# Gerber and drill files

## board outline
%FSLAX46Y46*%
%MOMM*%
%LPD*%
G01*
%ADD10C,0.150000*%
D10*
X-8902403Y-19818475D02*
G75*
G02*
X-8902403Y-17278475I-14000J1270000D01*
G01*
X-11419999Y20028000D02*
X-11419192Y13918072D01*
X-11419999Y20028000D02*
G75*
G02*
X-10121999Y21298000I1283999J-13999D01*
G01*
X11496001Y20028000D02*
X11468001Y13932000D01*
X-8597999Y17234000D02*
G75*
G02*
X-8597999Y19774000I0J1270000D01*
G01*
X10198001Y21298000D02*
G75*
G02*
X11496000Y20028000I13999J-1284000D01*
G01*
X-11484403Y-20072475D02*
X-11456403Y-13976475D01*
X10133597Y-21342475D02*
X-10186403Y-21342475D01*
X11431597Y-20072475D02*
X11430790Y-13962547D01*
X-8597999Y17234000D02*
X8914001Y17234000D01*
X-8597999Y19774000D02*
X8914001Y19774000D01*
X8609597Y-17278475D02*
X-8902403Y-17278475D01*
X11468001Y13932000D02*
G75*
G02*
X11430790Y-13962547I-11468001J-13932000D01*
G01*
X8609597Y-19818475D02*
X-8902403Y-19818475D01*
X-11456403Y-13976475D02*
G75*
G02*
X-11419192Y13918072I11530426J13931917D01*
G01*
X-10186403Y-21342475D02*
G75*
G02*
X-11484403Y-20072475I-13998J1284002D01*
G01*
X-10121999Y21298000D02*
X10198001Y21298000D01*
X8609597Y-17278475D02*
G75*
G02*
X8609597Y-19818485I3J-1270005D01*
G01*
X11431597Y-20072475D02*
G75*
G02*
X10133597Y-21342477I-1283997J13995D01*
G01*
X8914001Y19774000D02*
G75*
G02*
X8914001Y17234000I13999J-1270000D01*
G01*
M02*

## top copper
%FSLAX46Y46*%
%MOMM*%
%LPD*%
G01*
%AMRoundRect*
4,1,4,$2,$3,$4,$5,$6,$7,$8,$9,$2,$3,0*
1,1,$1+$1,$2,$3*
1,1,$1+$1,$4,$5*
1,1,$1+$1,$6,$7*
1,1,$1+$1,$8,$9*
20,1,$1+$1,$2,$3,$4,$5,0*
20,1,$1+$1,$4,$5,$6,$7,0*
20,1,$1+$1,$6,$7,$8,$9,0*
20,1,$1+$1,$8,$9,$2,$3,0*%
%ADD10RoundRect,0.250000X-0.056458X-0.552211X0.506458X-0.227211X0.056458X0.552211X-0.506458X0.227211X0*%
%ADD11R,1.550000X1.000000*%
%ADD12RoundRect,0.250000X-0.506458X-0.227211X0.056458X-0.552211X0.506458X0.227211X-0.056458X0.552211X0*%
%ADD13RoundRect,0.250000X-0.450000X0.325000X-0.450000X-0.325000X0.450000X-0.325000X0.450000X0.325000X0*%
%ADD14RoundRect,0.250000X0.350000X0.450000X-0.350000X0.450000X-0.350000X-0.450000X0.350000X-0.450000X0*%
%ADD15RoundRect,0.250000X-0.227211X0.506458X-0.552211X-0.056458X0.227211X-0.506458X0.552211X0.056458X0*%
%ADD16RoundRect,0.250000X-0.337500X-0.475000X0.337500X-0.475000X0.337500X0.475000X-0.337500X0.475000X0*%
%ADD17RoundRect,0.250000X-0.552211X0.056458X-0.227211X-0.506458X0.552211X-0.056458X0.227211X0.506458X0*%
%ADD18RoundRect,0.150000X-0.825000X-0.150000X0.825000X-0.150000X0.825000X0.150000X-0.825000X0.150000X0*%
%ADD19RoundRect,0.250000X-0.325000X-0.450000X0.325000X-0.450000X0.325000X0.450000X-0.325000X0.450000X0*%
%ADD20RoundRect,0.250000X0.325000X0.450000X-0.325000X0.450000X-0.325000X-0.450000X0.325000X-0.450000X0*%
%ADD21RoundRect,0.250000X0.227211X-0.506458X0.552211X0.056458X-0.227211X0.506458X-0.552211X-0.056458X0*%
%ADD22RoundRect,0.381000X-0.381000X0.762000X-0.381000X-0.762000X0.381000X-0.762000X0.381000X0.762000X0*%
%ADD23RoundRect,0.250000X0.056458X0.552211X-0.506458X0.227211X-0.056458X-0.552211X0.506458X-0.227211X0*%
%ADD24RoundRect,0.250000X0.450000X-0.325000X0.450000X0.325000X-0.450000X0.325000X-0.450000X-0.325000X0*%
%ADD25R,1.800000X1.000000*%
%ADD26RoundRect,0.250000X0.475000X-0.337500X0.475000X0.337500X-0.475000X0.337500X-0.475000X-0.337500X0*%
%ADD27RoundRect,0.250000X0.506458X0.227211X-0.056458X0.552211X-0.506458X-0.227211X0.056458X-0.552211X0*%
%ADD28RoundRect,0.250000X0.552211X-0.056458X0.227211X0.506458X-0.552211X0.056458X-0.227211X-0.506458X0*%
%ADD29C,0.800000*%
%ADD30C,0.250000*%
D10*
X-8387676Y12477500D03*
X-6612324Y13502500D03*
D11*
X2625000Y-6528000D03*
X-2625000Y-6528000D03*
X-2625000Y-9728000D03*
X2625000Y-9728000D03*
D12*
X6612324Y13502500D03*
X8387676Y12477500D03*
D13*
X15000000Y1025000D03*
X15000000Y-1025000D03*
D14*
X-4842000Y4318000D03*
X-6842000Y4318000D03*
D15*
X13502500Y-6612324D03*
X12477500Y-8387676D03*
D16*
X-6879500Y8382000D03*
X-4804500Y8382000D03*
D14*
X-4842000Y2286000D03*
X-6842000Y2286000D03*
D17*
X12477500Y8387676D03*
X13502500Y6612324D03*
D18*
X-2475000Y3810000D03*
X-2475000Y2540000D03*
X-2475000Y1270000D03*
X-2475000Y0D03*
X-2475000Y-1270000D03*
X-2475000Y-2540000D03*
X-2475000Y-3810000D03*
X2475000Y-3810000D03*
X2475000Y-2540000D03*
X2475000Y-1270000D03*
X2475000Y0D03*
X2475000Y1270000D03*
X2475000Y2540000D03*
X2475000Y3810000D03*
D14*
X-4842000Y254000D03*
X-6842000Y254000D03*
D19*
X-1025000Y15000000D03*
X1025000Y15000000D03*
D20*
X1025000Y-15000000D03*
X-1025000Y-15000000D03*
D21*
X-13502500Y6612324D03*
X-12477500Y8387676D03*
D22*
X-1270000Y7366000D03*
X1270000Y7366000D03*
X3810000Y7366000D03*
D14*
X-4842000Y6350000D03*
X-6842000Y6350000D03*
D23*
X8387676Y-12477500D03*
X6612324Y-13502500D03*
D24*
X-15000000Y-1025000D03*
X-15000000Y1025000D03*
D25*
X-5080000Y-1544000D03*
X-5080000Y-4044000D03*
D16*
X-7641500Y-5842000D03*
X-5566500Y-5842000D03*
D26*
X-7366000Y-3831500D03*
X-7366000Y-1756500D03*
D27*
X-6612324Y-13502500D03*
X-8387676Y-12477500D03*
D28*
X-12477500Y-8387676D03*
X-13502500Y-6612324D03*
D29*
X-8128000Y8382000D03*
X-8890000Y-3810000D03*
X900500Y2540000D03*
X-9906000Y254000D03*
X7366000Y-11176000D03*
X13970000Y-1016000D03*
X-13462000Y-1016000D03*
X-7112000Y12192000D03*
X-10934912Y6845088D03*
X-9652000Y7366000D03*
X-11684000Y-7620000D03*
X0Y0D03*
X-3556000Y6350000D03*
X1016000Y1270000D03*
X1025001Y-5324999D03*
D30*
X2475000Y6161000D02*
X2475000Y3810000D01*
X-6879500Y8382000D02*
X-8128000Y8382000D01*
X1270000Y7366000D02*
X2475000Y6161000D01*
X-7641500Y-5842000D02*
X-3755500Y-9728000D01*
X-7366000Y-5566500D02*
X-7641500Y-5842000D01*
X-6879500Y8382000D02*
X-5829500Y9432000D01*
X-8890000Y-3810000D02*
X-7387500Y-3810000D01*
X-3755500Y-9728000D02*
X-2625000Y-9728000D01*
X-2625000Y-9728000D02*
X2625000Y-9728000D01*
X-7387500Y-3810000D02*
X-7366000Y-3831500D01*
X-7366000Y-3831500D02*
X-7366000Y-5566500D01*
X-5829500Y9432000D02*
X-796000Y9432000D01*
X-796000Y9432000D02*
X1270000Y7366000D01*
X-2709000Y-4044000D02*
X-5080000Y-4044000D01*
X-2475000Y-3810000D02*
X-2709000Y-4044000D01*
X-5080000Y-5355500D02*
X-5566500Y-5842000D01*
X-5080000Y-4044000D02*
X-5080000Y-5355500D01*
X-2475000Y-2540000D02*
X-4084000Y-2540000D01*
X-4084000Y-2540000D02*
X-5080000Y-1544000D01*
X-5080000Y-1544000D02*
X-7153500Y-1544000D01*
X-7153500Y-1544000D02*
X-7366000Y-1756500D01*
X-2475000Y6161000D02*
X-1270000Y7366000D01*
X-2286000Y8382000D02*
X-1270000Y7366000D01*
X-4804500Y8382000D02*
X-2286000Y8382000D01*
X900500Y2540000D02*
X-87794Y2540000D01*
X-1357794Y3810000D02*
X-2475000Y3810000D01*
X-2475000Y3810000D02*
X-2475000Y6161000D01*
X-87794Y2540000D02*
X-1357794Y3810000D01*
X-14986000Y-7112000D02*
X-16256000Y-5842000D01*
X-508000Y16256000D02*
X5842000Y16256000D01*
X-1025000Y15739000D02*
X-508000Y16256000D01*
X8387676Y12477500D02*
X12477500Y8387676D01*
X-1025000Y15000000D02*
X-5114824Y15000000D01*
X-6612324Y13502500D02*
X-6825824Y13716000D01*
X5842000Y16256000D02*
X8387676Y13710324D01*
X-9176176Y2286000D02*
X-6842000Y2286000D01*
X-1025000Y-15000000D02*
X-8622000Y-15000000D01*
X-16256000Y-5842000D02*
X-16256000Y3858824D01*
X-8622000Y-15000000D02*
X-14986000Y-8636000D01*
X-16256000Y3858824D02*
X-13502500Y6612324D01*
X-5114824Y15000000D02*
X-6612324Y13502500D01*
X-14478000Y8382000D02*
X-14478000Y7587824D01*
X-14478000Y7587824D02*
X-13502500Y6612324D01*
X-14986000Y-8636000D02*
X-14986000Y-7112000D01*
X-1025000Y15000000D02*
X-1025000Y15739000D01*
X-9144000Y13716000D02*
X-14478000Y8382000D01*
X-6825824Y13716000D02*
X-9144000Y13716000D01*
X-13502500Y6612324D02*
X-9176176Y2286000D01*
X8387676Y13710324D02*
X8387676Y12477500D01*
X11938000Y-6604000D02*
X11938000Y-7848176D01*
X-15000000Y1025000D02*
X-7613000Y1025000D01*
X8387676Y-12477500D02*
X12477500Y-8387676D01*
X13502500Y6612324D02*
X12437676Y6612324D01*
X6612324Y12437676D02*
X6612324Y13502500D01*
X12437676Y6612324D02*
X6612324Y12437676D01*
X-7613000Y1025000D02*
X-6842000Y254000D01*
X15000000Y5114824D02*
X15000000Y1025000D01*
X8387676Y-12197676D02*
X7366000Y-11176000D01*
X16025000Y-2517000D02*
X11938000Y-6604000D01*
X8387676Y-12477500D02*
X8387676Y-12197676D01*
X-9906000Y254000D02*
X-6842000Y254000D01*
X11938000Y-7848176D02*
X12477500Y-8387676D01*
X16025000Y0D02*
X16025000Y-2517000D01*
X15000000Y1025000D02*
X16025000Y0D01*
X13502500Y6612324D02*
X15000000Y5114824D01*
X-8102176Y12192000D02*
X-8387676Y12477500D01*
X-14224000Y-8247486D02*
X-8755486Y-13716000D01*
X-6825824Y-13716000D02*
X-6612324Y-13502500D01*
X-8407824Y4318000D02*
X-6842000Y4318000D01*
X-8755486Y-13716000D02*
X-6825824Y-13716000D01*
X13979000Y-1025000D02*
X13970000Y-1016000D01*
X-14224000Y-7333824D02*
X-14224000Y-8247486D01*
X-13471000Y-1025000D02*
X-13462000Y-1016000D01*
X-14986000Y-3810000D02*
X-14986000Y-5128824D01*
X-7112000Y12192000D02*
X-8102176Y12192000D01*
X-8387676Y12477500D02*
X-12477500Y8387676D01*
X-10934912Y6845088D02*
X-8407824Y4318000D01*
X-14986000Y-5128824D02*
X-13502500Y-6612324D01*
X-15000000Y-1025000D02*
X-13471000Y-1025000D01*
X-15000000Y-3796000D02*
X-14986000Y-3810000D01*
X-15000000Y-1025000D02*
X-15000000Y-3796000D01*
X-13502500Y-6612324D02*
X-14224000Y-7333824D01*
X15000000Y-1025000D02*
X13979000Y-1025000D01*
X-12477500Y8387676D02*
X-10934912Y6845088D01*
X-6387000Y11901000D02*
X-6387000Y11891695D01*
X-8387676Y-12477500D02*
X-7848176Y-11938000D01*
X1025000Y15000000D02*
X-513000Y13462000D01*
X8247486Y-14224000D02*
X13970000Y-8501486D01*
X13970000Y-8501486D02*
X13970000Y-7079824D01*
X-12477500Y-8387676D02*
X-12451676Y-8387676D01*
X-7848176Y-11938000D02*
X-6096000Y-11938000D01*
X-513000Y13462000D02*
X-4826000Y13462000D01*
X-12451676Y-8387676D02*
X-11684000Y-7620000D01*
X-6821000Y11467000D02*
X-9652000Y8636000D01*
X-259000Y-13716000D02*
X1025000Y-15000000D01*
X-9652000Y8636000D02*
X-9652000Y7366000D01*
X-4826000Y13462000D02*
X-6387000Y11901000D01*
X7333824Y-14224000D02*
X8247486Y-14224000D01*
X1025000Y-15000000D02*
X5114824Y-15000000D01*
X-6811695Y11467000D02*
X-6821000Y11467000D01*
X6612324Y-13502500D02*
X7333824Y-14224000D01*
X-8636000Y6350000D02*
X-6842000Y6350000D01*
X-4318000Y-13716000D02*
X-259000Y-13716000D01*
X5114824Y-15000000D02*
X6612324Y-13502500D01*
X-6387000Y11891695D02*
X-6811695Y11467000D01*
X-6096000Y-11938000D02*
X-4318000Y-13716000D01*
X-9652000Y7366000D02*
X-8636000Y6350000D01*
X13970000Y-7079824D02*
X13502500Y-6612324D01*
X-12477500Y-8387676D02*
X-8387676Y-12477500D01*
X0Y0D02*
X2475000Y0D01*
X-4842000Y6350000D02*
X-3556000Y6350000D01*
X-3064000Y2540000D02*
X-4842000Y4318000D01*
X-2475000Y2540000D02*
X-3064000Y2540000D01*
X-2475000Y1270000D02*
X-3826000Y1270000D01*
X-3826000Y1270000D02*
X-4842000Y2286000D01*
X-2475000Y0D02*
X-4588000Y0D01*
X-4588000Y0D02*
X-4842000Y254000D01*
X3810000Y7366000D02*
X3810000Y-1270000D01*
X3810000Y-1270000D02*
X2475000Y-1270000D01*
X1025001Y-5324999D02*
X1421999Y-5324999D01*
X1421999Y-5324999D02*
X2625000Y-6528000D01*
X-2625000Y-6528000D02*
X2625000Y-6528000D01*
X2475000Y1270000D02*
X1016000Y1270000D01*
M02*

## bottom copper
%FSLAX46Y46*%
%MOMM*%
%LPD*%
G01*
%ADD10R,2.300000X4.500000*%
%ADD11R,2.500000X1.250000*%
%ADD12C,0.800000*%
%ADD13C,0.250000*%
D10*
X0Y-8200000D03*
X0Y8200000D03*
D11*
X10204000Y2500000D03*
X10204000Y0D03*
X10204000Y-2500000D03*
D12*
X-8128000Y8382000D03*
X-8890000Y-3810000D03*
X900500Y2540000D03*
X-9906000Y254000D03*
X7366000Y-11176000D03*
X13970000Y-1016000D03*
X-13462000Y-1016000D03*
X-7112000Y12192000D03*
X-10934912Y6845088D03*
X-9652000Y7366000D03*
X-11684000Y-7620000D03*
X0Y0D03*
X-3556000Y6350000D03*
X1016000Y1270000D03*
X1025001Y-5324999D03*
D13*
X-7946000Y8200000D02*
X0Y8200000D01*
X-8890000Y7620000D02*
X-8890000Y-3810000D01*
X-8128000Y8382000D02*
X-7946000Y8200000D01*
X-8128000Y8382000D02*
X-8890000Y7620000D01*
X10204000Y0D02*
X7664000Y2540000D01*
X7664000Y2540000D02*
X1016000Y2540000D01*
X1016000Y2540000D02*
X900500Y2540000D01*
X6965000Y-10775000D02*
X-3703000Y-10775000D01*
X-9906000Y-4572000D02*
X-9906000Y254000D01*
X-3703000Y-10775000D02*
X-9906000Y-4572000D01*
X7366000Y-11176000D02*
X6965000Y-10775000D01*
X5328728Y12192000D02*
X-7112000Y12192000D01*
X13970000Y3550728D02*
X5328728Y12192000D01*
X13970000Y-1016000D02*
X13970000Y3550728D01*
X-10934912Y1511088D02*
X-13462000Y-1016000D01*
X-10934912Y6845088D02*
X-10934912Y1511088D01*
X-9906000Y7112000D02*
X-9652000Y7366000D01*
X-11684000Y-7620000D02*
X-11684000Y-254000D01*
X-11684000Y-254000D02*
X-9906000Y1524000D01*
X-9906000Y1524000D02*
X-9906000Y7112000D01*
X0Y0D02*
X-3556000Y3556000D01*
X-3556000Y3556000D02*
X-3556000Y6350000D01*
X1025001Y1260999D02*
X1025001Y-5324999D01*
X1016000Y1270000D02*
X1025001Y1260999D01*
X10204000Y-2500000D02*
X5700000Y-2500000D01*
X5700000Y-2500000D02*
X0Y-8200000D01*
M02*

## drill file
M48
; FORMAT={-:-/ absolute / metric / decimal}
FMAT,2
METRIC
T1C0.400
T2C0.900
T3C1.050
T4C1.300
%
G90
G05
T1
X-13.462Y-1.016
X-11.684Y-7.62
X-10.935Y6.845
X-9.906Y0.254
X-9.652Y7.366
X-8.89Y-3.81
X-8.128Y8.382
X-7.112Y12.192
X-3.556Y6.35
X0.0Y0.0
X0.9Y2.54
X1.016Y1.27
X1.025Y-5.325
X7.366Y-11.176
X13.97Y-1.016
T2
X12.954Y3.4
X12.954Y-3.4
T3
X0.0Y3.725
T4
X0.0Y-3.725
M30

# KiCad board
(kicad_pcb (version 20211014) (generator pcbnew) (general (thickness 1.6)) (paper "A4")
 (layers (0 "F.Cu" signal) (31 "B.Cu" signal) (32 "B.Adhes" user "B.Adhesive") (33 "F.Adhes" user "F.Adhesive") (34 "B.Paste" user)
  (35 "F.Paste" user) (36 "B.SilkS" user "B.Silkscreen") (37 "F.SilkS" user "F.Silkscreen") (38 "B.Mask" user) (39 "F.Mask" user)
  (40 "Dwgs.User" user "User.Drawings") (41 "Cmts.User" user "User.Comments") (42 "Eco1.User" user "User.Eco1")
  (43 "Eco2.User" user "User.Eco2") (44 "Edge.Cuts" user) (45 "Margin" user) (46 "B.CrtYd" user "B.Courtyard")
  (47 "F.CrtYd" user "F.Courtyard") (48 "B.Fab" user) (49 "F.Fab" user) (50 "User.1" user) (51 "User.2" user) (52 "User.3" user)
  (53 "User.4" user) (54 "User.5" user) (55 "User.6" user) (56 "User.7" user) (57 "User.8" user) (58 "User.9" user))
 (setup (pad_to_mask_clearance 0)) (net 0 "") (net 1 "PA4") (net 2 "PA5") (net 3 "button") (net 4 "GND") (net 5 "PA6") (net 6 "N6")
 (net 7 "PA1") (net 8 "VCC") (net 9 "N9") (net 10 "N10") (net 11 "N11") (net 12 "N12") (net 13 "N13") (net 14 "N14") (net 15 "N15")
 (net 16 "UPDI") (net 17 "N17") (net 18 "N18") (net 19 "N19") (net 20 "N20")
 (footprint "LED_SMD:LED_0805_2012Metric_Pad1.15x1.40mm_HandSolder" (layer "F.Cu") (at -7.5 -12.99 30)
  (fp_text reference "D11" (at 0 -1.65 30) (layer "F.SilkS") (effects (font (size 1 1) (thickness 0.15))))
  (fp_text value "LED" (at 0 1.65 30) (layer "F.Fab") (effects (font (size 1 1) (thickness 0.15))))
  (pad "1" smd roundrect (at -1.025 0 30) (size 1.15 1.4) (layers "F.Cu" "F.Paste" "F.Mask") (roundrect_rratio 0.217391) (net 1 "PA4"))
  (pad "2" smd roundrect (at 1.025 0 30) (size 1.15 1.4) (layers "F.Cu" "F.Paste" "F.Mask") (roundrect_rratio 0.217391) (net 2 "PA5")))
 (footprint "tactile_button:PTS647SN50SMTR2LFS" (layer "F.Cu") (at 0 8.128 180)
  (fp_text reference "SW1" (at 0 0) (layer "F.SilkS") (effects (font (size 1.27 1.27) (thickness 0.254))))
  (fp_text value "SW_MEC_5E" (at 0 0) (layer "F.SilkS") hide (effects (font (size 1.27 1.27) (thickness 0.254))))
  (pad "1" smd rect locked (at -2.625 1.6 270) (size 1 1.55) (layers "F.Cu" "F.Paste" "F.Mask") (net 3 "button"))
  (pad "2" smd rect locked (at 2.625 1.6 270) (size 1 1.55) (layers "F.Cu" "F.Paste" "F.Mask") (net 3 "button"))
  (pad "3" smd rect locked (at 2.625 -1.6 270) (size 1 1.55) (layers "F.Cu" "F.Paste" "F.Mask") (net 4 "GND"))
  (pad "4" smd rect locked (at -2.625 -1.6 270) (size 1 1.55) (layers "F.Cu" "F.Paste" "F.Mask") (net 4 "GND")))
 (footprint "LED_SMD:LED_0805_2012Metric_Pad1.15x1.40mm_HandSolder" (layer "F.Cu") (at 7.5 -12.99 -30)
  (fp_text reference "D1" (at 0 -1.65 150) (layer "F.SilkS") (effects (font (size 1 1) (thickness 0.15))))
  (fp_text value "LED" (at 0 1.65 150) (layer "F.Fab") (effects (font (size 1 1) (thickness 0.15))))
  (pad "1" smd roundrect (at -1.025 0 330) (size 1.15 1.4) (layers "F.Cu" "F.Paste" "F.Mask") (roundrect_rratio 0.217391) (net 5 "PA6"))
  (pad "2" smd roundrect (at 1.025 0 330) (size 1.15 1.4) (layers "F.Cu" "F.Paste" "F.Mask") (roundrect_rratio 0.217391) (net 2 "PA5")))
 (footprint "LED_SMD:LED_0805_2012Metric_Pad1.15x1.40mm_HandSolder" (layer "F.Cu") (at 15 0 -90)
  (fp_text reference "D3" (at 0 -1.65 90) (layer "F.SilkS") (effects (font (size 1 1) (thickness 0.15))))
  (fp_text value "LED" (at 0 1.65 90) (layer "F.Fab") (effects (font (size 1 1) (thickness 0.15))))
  (pad "1" smd roundrect (at -1.025 0 270) (size 1.15 1.4) (layers "F.Cu" "F.Paste" "F.Mask") (roundrect_rratio 0.217391) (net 5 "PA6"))
  (pad "2" smd roundrect (at 1.025 0 270) (size 1.15 1.4) (layers "F.Cu" "F.Paste" "F.Mask") (roundrect_rratio 0.217391) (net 1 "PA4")))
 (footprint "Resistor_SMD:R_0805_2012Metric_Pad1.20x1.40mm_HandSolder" (layer "F.Cu") (at -5.842 -4.318 180)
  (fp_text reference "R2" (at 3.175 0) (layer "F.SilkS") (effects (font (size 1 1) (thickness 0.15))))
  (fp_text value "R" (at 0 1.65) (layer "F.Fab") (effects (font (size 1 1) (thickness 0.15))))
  (pad "1" smd roundrect (at -1 0 180) (size 1.2 1.4) (layers "F.Cu" "F.Paste" "F.Mask") (roundrect_rratio 0.208333) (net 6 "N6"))
  (pad "2" smd roundrect (at 1 0 180) (size 1.2 1.4) (layers "F.Cu" "F.Paste" "F.Mask") (roundrect_rratio 0.208333) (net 1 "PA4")))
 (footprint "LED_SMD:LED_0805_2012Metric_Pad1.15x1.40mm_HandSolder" (layer "F.Cu") (at 12.99 7.5 -120)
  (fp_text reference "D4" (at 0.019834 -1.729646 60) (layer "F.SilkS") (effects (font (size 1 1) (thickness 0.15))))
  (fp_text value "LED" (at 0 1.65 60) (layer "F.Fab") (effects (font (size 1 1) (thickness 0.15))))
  (pad "1" smd roundrect (at -1.025 0 240) (size 1.15 1.4) (layers "F.Cu" "F.Paste" "F.Mask") (roundrect_rratio 0.217391) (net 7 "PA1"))
  (pad "2" smd roundrect (at 1.025 0 240) (size 1.15 1.4) (layers "F.Cu" "F.Paste" "F.Mask") (roundrect_rratio 0.217391) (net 5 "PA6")))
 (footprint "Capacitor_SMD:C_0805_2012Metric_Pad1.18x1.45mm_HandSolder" (layer "F.Cu") (at -5.842 -8.382)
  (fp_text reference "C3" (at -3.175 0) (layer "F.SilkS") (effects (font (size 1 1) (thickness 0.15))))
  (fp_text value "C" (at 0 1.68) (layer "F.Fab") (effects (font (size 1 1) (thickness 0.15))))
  (pad "1" smd roundrect (at -1.0375 0) (size 1.175 1.45) (layers "F.Cu" "F.Paste" "F.Mask") (roundrect_rratio 0.212766) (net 4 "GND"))
  (pad "2" smd roundrect (at 1.0375 0) (size 1.175 1.45) (layers "F.Cu" "F.Paste" "F.Mask") (roundrect_rratio 0.212766) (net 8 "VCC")))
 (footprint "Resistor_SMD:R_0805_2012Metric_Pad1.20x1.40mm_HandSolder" (layer "F.Cu") (at -5.842 -2.286 180)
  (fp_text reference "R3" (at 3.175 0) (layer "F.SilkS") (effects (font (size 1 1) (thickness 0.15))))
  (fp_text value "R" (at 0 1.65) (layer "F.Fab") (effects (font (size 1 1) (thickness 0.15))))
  (pad "1" smd roundrect (at -1 0 180) (size 1.2 1.4) (layers "F.Cu" "F.Paste" "F.Mask") (roundrect_rratio 0.208333) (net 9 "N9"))
  (pad "2" smd roundrect (at 1 0 180) (size 1.2 1.4) (layers "F.Cu" "F.Paste" "F.Mask") (roundrect_rratio 0.208333) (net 2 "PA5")))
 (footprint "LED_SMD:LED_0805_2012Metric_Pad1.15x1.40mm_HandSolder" (layer "F.Cu") (at 12.99 -7.5 -60)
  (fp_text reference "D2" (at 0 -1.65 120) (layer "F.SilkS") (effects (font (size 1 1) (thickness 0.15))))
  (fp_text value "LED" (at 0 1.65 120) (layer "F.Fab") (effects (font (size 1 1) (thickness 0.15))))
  (pad "1" smd roundrect (at -1.025 0 300) (size 1.15 1.4) (layers "F.Cu" "F.Paste" "F.Mask") (roundrect_rratio 0.217391) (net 2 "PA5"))
  (pad "2" smd roundrect (at 1.025 0 300) (size 1.15 1.4) (layers "F.Cu" "F.Paste" "F.Mask") (roundrect_rratio 0.217391) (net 5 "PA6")))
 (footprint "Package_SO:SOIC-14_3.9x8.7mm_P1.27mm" (layer "F.Cu") (at 0 0)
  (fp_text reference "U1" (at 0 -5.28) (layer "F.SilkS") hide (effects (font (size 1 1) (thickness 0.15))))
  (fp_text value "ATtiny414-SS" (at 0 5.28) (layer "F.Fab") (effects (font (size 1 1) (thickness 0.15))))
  (pad "1" smd roundrect (at -2.475 -3.81) (size 1.95 0.6) (layers "F.Cu" "F.Paste" "F.Mask") (roundrect_rratio 0.25) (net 8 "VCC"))
  (pad "2" smd roundrect (at -2.475 -2.54) (size 1.95 0.6) (layers "F.Cu" "F.Paste" "F.Mask") (roundrect_rratio 0.25) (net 6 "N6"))
  (pad "3" smd roundrect (at -2.475 -1.27) (size 1.95 0.6) (layers "F.Cu" "F.Paste" "F.Mask") (roundrect_rratio 0.25) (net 9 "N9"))
  (pad "4" smd roundrect (at -2.475 0) (size 1.95 0.6) (layers "F.Cu" "F.Paste" "F.Mask") (roundrect_rratio 0.25) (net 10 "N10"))
  (pad "5" smd roundrect (at -2.475 1.27) (size 1.95 0.6) (layers "F.Cu" "F.Paste" "F.Mask") (roundrect_rratio 0.25) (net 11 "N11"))
  (pad "6" smd roundrect (at -2.475 2.54) (size 1.95 0.6) (layers "F.Cu" "F.Paste" "F.Mask") (roundrect_rratio 0.25) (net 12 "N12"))
  (pad "7" smd roundrect (at -2.475 3.81) (size 1.95 0.6) (layers "F.Cu" "F.Paste" "F.Mask") (roundrect_rratio 0.25) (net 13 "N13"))
  (pad "8" smd roundrect (at 2.475 3.81) (size 1.95 0.6) (layers "F.Cu" "F.Paste" "F.Mask") (roundrect_rratio 0.25) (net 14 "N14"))
  (pad "9" smd roundrect (at 2.475 2.54) (size 1.95 0.6) (layers "F.Cu" "F.Paste" "F.Mask") (roundrect_rratio 0.25) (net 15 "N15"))
  (pad "10" smd roundrect (at 2.475 1.27) (size 1.95 0.6) (layers "F.Cu" "F.Paste" "F.Mask") (roundrect_rratio 0.25) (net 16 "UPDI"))
  (pad "11" smd roundrect (at 2.475 0) (size 1.95 0.6) (layers "F.Cu" "F.Paste" "F.Mask") (roundrect_rratio 0.25) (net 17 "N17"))
  (pad "12" smd roundrect (at 2.475 -1.27) (size 1.95 0.6) (layers "F.Cu" "F.Paste" "F.Mask") (roundrect_rratio 0.25) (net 3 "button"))
  (pad "13" smd roundrect (at 2.475 -2.54) (size 1.95 0.6) (layers "F.Cu" "F.Paste" "F.Mask") (roundrect_rratio 0.25) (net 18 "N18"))
  (pad "14" smd roundrect (at 2.475 -3.81) (size 1.95 0.6) (layers "F.Cu" "F.Paste" "F.Mask") (roundrect_rratio 0.25) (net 4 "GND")))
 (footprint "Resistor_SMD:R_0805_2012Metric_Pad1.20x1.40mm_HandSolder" (layer "F.Cu") (at -5.842 -0.254 180)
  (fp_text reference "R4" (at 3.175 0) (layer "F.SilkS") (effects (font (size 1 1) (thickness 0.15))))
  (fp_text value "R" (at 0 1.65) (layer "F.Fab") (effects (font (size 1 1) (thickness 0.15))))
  (pad "1" smd roundrect (at -1 0 180) (size 1.2 1.4) (layers "F.Cu" "F.Paste" "F.Mask") (roundrect_rratio 0.208333) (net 10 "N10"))
  (pad "2" smd roundrect (at 1 0 180) (size 1.2 1.4) (layers "F.Cu" "F.Paste" "F.Mask") (roundrect_rratio 0.208333) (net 5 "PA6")))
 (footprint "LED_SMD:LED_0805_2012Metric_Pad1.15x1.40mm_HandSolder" (layer "F.Cu") (at 0 -15)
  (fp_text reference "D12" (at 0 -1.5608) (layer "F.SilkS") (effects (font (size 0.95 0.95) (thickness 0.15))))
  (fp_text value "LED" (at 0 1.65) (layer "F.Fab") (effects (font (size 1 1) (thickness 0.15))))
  (pad "1" smd roundrect (at -1.025 0) (size 1.15 1.4) (layers "F.Cu" "F.Paste" "F.Mask") (roundrect_rratio 0.217391) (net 2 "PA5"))
  (pad "2" smd roundrect (at 1.025 0) (size 1.15 1.4) (layers "F.Cu" "F.Paste" "F.Mask") (roundrect_rratio 0.217391) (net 7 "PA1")))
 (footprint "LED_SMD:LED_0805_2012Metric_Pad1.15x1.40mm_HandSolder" (layer "F.Cu") (at 0 15 180)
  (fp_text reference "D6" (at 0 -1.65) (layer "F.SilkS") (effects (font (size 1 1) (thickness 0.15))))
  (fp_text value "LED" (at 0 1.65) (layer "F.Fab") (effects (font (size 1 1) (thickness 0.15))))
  (pad "1" smd roundrect (at -1.025 0 180) (size 1.15 1.4) (layers "F.Cu" "F.Paste" "F.Mask") (roundrect_rratio 0.217391) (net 7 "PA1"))
  (pad "2" smd roundrect (at 1.025 0 180) (size 1.15 1.4) (layers "F.Cu" "F.Paste" "F.Mask") (roundrect_rratio 0.217391) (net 2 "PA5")))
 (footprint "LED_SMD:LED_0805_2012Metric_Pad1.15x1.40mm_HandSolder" (layer "F.Cu") (at -12.99 -7.5 60)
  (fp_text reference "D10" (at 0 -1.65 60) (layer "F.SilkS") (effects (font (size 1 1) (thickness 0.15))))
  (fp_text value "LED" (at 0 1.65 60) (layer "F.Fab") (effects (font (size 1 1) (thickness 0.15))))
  (pad "1" smd roundrect (at -1.025 0 60) (size 1.15 1.4) (layers "F.Cu" "F.Paste" "F.Mask") (roundrect_rratio 0.217391) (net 2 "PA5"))
  (pad "2" smd roundrect (at 1.025 0 60) (size 1.15 1.4) (layers "F.Cu" "F.Paste" "F.Mask") (roundrect_rratio 0.217391) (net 1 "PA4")))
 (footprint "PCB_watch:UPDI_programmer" (layer "F.Cu") (at 1.27 -7.366 -90)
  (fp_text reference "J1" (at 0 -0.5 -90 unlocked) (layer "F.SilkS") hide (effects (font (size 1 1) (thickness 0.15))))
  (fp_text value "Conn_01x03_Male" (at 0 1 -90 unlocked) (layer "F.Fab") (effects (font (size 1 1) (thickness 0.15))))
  (pad "1" smd roundrect (at 0 2.54 270) (size 2.286 1.524) (layers "F.Cu" "F.Paste" "F.Mask") (roundrect_rratio 0.25) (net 8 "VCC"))
  (pad "2" smd roundrect (at 0 0 270) (size 2.286 1.524) (layers "F.Cu" "F.Paste" "F.Mask") (roundrect_rratio 0.25) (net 4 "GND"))
  (pad "3" smd roundrect (at 0 -2.54 270) (size 2.286 1.524) (layers "F.Cu" "F.Paste" "F.Mask") (roundrect_rratio 0.25) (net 16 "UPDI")))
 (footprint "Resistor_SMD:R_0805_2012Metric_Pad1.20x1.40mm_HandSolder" (layer "F.Cu") (at -5.842 -6.35 180)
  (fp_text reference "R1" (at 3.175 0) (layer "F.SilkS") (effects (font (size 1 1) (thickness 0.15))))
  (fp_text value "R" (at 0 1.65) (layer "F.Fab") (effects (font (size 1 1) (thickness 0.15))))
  (pad "1" smd roundrect (at -1 0 180) (size 1.2 1.4) (layers "F.Cu" "F.Paste" "F.Mask") (roundrect_rratio 0.208333) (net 17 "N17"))
  (pad "2" smd roundrect (at 1 0 180) (size 1.2 1.4) (layers "F.Cu" "F.Paste" "F.Mask") (roundrect_rratio 0.208333) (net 7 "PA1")))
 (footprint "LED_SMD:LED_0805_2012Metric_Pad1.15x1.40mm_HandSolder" (layer "F.Cu") (at 7.5 12.99 -150)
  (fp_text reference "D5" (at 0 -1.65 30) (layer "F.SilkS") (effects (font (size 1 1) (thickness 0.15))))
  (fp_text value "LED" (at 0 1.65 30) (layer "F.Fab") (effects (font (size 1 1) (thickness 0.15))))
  (pad "1" smd roundrect (at -1.025 0 210) (size 1.15 1.4) (layers "F.Cu" "F.Paste" "F.Mask") (roundrect_rratio 0.217391) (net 5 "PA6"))
  (pad "2" smd roundrect (at 1.025 0 210) (size 1.15 1.4) (layers "F.Cu" "F.Paste" "F.Mask") (roundrect_rratio 0.217391) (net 7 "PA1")))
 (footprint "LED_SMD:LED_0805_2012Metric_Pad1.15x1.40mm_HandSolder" (layer "F.Cu") (at -15 0 90)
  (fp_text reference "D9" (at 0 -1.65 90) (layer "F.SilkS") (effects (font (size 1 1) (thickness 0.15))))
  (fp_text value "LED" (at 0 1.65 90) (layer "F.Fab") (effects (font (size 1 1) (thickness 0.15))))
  (pad "1" smd roundrect (at -1.025 0 90) (size 1.15 1.4) (layers "F.Cu" "F.Paste" "F.Mask") (roundrect_rratio 0.217391) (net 1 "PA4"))
  (pad "2" smd roundrect (at 1.025 0 90) (size 1.15 1.4) (layers "F.Cu" "F.Paste" "F.Mask") (roundrect_rratio 0.217391) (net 5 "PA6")))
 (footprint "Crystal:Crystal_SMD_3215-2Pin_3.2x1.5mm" (layer "F.Cu") (at -5.08 2.794 90)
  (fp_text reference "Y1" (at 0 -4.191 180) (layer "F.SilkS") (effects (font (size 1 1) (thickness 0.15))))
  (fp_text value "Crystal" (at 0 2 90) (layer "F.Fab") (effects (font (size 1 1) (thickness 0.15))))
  (pad "1" smd rect (at 1.25 0 90) (size 1 1.8) (layers "F.Cu" "F.Paste" "F.Mask") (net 12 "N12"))
  (pad "2" smd rect (at -1.25 0 90) (size 1 1.8) (layers "F.Cu" "F.Paste" "F.Mask") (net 13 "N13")))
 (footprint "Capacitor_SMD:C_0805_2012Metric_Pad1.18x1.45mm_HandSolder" (layer "F.Cu") (at -6.604 5.842)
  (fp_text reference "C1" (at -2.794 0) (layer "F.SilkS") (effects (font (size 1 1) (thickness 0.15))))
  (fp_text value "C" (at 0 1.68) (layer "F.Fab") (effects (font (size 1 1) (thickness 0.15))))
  (pad "1" smd roundrect (at -1.0375 0) (size 1.175 1.45) (layers "F.Cu" "F.Paste" "F.Mask") (roundrect_rratio 0.212766) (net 4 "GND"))
  (pad "2" smd roundrect (at 1.0375 0) (size 1.175 1.45) (layers "F.Cu" "F.Paste" "F.Mask") (roundrect_rratio 0.212766) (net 13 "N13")))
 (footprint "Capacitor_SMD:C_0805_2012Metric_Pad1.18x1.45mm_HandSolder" (layer "F.Cu") (at -7.366 2.794 90)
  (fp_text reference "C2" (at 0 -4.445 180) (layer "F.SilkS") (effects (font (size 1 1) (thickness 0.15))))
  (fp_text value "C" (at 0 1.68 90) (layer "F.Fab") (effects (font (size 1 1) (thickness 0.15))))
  (pad "1" smd roundrect (at -1.0375 0 90) (size 1.175 1.45) (layers "F.Cu" "F.Paste" "F.Mask") (roundrect_rratio 0.212766) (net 4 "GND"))
  (pad "2" smd roundrect (at 1.0375 0 90) (size 1.175 1.45) (layers "F.Cu" "F.Paste" "F.Mask") (roundrect_rratio 0.212766) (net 12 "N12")))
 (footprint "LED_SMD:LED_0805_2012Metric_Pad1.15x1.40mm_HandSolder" (layer "F.Cu") (at -7.5 12.99 150)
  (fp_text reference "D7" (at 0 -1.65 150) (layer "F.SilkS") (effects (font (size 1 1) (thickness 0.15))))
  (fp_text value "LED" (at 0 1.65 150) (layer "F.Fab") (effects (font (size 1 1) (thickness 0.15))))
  (pad "1" smd roundrect (at -1.025 0 150) (size 1.15 1.4) (layers "F.Cu" "F.Paste" "F.Mask") (roundrect_rratio 0.217391) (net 1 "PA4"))
  (pad "2" smd roundrect (at 1.025 0 150) (size 1.15 1.4) (layers "F.Cu" "F.Paste" "F.Mask") (roundrect_rratio 0.217391) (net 7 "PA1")))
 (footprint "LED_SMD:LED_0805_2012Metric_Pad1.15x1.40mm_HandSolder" (layer "F.Cu") (at -12.99 7.5 120)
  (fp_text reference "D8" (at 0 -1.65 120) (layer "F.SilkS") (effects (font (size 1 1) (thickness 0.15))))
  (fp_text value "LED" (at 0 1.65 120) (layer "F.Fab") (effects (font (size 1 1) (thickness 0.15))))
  (pad "1" smd roundrect (at -1.025 0 120) (size 1.15 1.4) (layers "F.Cu" "F.Paste" "F.Mask") (roundrect_rratio 0.217391) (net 7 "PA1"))
  (pad "2" smd roundrect (at 1.025 0 120) (size 1.15 1.4) (layers "F.Cu" "F.Paste" "F.Mask") (roundrect_rratio 0.217391) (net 1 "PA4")))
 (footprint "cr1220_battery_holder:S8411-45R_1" (layer "B.Cu") (at 0 0 180)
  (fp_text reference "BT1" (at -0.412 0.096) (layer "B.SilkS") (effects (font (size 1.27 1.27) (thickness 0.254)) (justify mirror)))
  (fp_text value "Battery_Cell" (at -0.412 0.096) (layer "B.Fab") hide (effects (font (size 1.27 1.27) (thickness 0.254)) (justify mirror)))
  (pad "" np_thru_hole circle locked (at 0 3.725 180) (size 0.001 0.001) (drill 1.05) (layers *.Cu *.Mask))
  (pad "" np_thru_hole circle locked (at 0 -3.725 180) (size 0.001 0.001) (drill 1.3) (layers *.Cu *.Mask))
  (pad "1" smd rect locked (at 0 -8.2 180) (size 2.3 4.5) (layers "B.Cu" "B.Paste" "B.Mask") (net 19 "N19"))
  (pad "2" smd rect locked (at 0 8.2 180) (size 2.3 4.5) (layers "B.Cu" "B.Paste" "B.Mask") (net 4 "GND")))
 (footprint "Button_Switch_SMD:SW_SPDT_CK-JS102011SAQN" (layer "B.Cu") (at 12.954 0 -90)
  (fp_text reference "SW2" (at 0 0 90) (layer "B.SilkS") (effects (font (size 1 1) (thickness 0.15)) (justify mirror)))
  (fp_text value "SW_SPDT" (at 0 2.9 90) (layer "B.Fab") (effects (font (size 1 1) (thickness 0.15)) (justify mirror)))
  (pad "" np_thru_hole circle (at -3.4 0 270) (size 0.9 0.9) (drill 0.9) (layers *.Cu *.Mask))
  (pad "" np_thru_hole circle (at 3.4 0 270) (size 0.9 0.9) (drill 0.9) (layers *.Cu *.Mask))
  (pad "1" smd rect (at -2.5 2.75 270) (size 1.25 2.5) (layers "B.Cu" "B.Paste" "B.Mask") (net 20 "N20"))
  (pad "2" smd rect (at 0 2.75 270) (size 1.25 2.5) (layers "B.Cu" "B.Paste" "B.Mask") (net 8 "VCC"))
  (pad "3" smd rect (at 2.5 2.75 270) (size 1.25 2.5) (layers "B.Cu" "B.Paste" "B.Mask") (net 19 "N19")))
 (gr_arc (start -8.902403 19.818475) (mid -10.18648 18.548475) (end -8.902403 17.278475) (layer "Edge.Cuts") (width 0.15))
 (gr_line (start -11.419999 -20.028) (end -11.419192 -13.918072) (layer "Edge.Cuts") (width 0.15))
 (gr_arc (start -11.419999 -20.028) (mid -11.034025 -20.931825) (end -10.121999 -21.298) (layer "Edge.Cuts") (width 0.15))
 (gr_line (start 11.496001 -20.028) (end 11.468001 -13.932) (layer "Edge.Cuts") (width 0.15))
 (gr_arc (start -8.597999 -17.234) (mid -9.867999 -18.504) (end -8.597999 -19.774) (layer "Edge.Cuts") (width 0.15))
 (gr_arc (start 10.198001 -21.298) (mid 11.110026 -20.931824) (end 11.496001 -20.028) (layer "Edge.Cuts") (width 0.15))
 (gr_line (start -11.484403 20.072475) (end -11.456403 13.976475) (layer "Edge.Cuts") (width 0.15))
 (gr_line (start 10.133597 21.342475) (end -10.186403 21.342475) (layer "Edge.Cuts") (width 0.15))
 (gr_line (start 11.431597 20.072475) (end 11.43079 13.962547) (layer "Edge.Cuts") (width 0.15))
 (gr_line (start -8.597999 -17.234) (end 8.914001 -17.234) (layer "Edge.Cuts") (width 0.15))
 (gr_line (start -8.597999 -19.774) (end 8.914001 -19.774) (layer "Edge.Cuts") (width 0.15))
 (gr_line (start 8.609597 17.278475) (end -8.902403 17.278475) (layer "Edge.Cuts") (width 0.15))
 (gr_arc (start 11.468001 -13.932) (mid 18.044808 0.024072) (end 11.43079 13.962547) (layer "Edge.Cuts") (width 0.15))
 (gr_line (start 8.609597 19.818475) (end -8.902403 19.818475) (layer "Edge.Cuts") (width 0.15))
 (gr_arc (start -11.456403 13.976475) (mid -18.010458 0.020434) (end -11.419192 -13.918072) (layer "Edge.Cuts") (width 0.15))
 (gr_arc (start -10.186403 21.342475) (mid -11.098428 20.976299) (end -11.484403 20.072475) (layer "Edge.Cuts") (width 0.15))
 (gr_line (start -10.121999 -21.298) (end 10.198001 -21.298) (layer "Edge.Cuts") (width 0.15))
 (gr_arc (start 8.609597 17.278475) (mid 9.879597 18.548475) (end 8.609597 19.818475) (layer "Edge.Cuts") (width 0.15))
 (gr_arc (start 11.431597 20.072475) (mid 11.045623 20.9763) (end 10.133597 21.342475) (layer "Edge.Cuts") (width 0.15))
 (gr_arc (start 8.914001 -19.774) (mid 10.198078 -18.504) (end 8.914001 -17.234) (layer "Edge.Cuts") (width 0.15))
 (segment (start 2.475 -6.161) (end 2.475 -3.81) (width 0.25) (layer "F.Cu") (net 4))
 (segment (start -6.8795 -8.382) (end -8.128 -8.382) (width 0.25) (layer "F.Cu") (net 4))
 (segment (start 1.27 -7.366) (end 2.475 -6.161) (width 0.25) (layer "F.Cu") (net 4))
 (segment (start -7.6415 5.842) (end -3.7555 9.728) (width 0.25) (layer "F.Cu") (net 4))
 (segment (start -7.366 5.5665) (end -7.6415 5.842) (width 0.25) (layer "F.Cu") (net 4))
 (segment (start -6.8795 -8.382) (end -5.8295 -9.432) (width 0.25) (layer "F.Cu") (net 4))
 (segment (start -8.89 3.81) (end -7.3875 3.81) (width 0.25) (layer "F.Cu") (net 4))
 (segment (start -3.7555 9.728) (end -2.625 9.728) (width 0.25) (layer "F.Cu") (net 4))
 (segment (start -2.625 9.728) (end 2.625 9.728) (width 0.25) (layer "F.Cu") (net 4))
 (segment (start -7.3875 3.81) (end -7.366 3.8315) (width 0.25) (layer "F.Cu") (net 4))
 (segment (start -7.366 3.8315) (end -7.366 5.5665) (width 0.25) (layer "F.Cu") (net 4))
 (segment (start -5.8295 -9.432) (end -0.796 -9.432) (width 0.25) (layer "F.Cu") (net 4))
 (segment (start -0.796 -9.432) (end 1.27 -7.366) (width 0.25) (layer "F.Cu") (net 4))
 (via (at -8.128 -8.382) (size 0.8) (drill 0.4) (layers "F.Cu" "B.Cu") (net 4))
 (via (at -8.89 3.81) (size 0.8) (drill 0.4) (layers "F.Cu" "B.Cu") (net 4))
 (segment (start -7.946 -8.2) (end 0 -8.2) (width 0.25) (layer "B.Cu") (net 4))
 (segment (start -8.89 -7.62) (end -8.89 3.81) (width 0.25) (layer "B.Cu") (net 4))
 (segment (start -8.128 -8.382) (end -7.946 -8.2) (width 0.25) (layer "B.Cu") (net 4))
 (segment (start -8.128 -8.382) (end -8.89 -7.62) (width 0.25) (layer "B.Cu") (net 4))
 (segment (start -2.709 4.044) (end -5.08 4.044) (width 0.25) (layer "F.Cu") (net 13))
 (segment (start -2.475 3.81) (end -2.709 4.044) (width 0.25) (layer "F.Cu") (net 13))
 (segment (start -5.08 5.3555) (end -5.5665 5.842) (width 0.25) (layer "F.Cu") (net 13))
 (segment (start -5.08 4.044) (end -5.08 5.3555) (width 0.25) (layer "F.Cu") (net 13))
 (segment (start -2.475 2.54) (end -4.084 2.54) (width 0.25) (layer "F.Cu") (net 12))
 (segment (start -4.084 2.54) (end -5.08 1.544) (width 0.25) (layer "F.Cu") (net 12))
 (segment (start -5.08 1.544) (end -7.1535 1.544) (width 0.25) (layer "F.Cu") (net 12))
 (segment (start -7.1535 1.544) (end -7.366 1.7565) (width 0.25) (layer "F.Cu") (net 12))
 (segment (start -2.475 -6.161) (end -1.27 -7.366) (width 0.25) (layer "F.Cu") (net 8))
 (segment (start -2.286 -8.382) (end -1.27 -7.366) (width 0.25) (layer "F.Cu") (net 8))
 (segment (start -4.8045 -8.382) (end -2.286 -8.382) (width 0.25) (layer "F.Cu") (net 8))
 (segment (start 0.9005 -2.54) (end -0.087794 -2.54) (width 0.25) (layer "F.Cu") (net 8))
 (segment (start -1.357794 -3.81) (end -2.475 -3.81) (width 0.25) (layer "F.Cu") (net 8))
 (segment (start -2.475 -3.81) (end -2.475 -6.161) (width 0.25) (layer "F.Cu") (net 8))
 (segment (start -0.087794 -2.54) (end -1.357794 -3.81) (width 0.25) (layer "F.Cu") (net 8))
 (via (at 0.9005 -2.54) (size 0.8) (drill 0.4) (layers "F.Cu" "B.Cu") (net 8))
 (segment (start 10.204 0) (end 7.664 -2.54) (width 0.25) (layer "B.Cu") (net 8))
 (segment (start 7.664 -2.54) (end 1.016 -2.54) (width 0.25) (layer "B.Cu") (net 8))
 (segment (start 1.016 -2.54) (end 0.9005 -2.54) (width 0.25) (layer "B.Cu") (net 8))
 (segment (start -14.986 7.112) (end -16.256 5.842) (width 0.25) (layer "F.Cu") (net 2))
 (segment (start -0.508 -16.256) (end 5.842 -16.256) (width 0.25) (layer "F.Cu") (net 2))
 (segment (start -1.025 -15.739) (end -0.508 -16.256) (width 0.25) (layer "F.Cu") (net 2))
 (segment (start 8.387676 -12.4775) (end 12.4775 -8.387676) (width 0.25) (layer "F.Cu") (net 2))
 (segment (start -1.025 -15) (end -5.114824 -15) (width 0.25) (layer "F.Cu") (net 2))
 (segment (start -6.612324 -13.5025) (end -6.825824 -13.716) (width 0.25) (layer "F.Cu") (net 2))
 (segment (start 5.842 -16.256) (end 8.387676 -13.710324) (width 0.25) (layer "F.Cu") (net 2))
 (segment (start -9.176176 -2.286) (end -6.842 -2.286) (width 0.25) (layer "F.Cu") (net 2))
 (segment (start -1.025 15) (end -8.622 15) (width 0.25) (layer "F.Cu") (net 2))
 (segment (start -16.256 5.842) (end -16.256 -3.858824) (width 0.25) (layer "F.Cu") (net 2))
 (segment (start -8.622 15) (end -14.986 8.636) (width 0.25) (layer "F.Cu") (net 2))
 (segment (start -16.256 -3.858824) (end -13.5025 -6.612324) (width 0.25) (layer "F.Cu") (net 2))
 (segment (start -5.114824 -15) (end -6.612324 -13.5025) (width 0.25) (layer "F.Cu") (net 2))
 (segment (start -14.478 -8.382) (end -14.478 -7.587824) (width 0.25) (layer "F.Cu") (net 2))
 (segment (start -14.478 -7.587824) (end -13.5025 -6.612324) (width 0.25) (layer "F.Cu") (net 2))
 (segment (start -14.986 8.636) (end -14.986 7.112) (width 0.25) (layer "F.Cu") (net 2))
 (segment (start -1.025 -15) (end -1.025 -15.739) (width 0.25) (layer "F.Cu") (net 2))
 (segment (start -9.144 -13.716) (end -14.478 -8.382) (width 0.25) (layer "F.Cu") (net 2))
 (segment (start -6.825824 -13.716) (end -9.144 -13.716) (width 0.25) (layer "F.Cu") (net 2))
 (segment (start -13.5025 -6.612324) (end -9.176176 -2.286) (width 0.25) (layer "F.Cu") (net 2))
 (segment (start 8.387676 -13.710324) (end 8.387676 -12.4775) (width 0.25) (layer "F.Cu") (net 2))
 (segment (start 11.938 6.604) (end 11.938 7.848176) (width 0.25) (layer "F.Cu") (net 5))
 (segment (start -15 -1.025) (end -7.613 -1.025) (width 0.25) (layer "F.Cu") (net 5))
 (segment (start 8.387676 12.4775) (end 12.4775 8.387676) (width 0.25) (layer "F.Cu") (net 5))
 (segment (start 13.5025 -6.612324) (end 12.437676 -6.612324) (width 0.25) (layer "F.Cu") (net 5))
 (segment (start 6.612324 -12.437676) (end 6.612324 -13.5025) (width 0.25) (layer "F.Cu") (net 5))
 (segment (start 12.437676 -6.612324) (end 6.612324 -12.437676) (width 0.25) (layer "F.Cu") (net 5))
 (segment (start -7.613 -1.025) (end -6.842 -0.254) (width 0.25) (layer "F.Cu") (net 5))
 (segment (start 15 -5.114824) (end 15 -1.025) (width 0.25) (layer "F.Cu") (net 5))
 (segment (start 8.387676 12.197676) (end 7.366 11.176) (width 0.25) (layer "F.Cu") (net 5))
 (segment (start 16.025 2.517) (end 11.938 6.604) (width 0.25) (layer "F.Cu") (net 5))
 (segment (start 8.387676 12.4775) (end 8.387676 12.197676) (width 0.25) (layer "F.Cu") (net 5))
 (segment (start -9.906 -0.254) (end -6.842 -0.254) (width 0.25) (layer "F.Cu") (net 5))
 (segment (start 11.938 7.848176) (end 12.4775 8.387676) (width 0.25) (layer "F.Cu") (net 5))
 (segment (start 16.025 0) (end 16.025 2.517) (width 0.25) (layer "F.Cu") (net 5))
 (segment (start 15 -1.025) (end 16.025 0) (width 0.25) (layer "F.Cu") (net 5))
 (segment (start 13.5025 -6.612324) (end 15 -5.114824) (width 0.25) (layer "F.Cu") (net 5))
 (via (at -9.906 -0.254) (size 0.8) (drill 0.4) (layers "F.Cu" "B.Cu") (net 5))
 (via (at 7.366 11.176) (size 0.8) (drill 0.4) (layers "F.Cu" "B.Cu") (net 5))
 (segment (start 6.965 10.775) (end -3.703 10.775) (width 0.25) (layer "B.Cu") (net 5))
 (segment (start -9.906 4.572) (end -9.906 -0.254) (width 0.25) (layer "B.Cu") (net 5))
 (segment (start -3.703 10.775) (end -9.906 4.572) (width 0.25) (layer "B.Cu") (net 5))
 (segment (start 7.366 11.176) (end 6.965 10.775) (width 0.25) (layer "B.Cu") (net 5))
 (segment (start -8.102176 -12.192) (end -8.387676 -12.4775) (width 0.25) (layer "F.Cu") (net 1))
 (segment (start -14.224 8.247486) (end -8.755486 13.716) (width 0.25) (layer "F.Cu") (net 1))
 (segment (start -6.825824 13.716) (end -6.612324 13.5025) (width 0.25) (layer "F.Cu") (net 1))
 (segment (start -8.407824 -4.318) (end -6.842 -4.318) (width 0.25) (layer "F.Cu") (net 1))
 (segment (start -8.755486 13.716) (end -6.825824 13.716) (width 0.25) (layer "F.Cu") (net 1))
 (segment (start 13.979 1.025) (end 13.97 1.016) (width 0.25) (layer "F.Cu") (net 1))
 (segment (start -14.224 7.333824) (end -14.224 8.247486) (width 0.25) (layer "F.Cu") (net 1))
 (segment (start -13.471 1.025) (end -13.462 1.016) (width 0.25) (layer "F.Cu") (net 1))
 (segment (start -14.986 3.81) (end -14.986 5.128824) (width 0.25) (layer "F.Cu") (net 1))
 (segment (start -7.112 -12.192) (end -8.102176 -12.192) (width 0.25) (layer "F.Cu") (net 1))
 (segment (start -8.387676 -12.4775) (end -12.4775 -8.387676) (width 0.25) (layer "F.Cu") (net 1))
 (segment (start -10.934912 -6.845088) (end -8.407824 -4.318) (width 0.25) (layer "F.Cu") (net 1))
 (segment (start -14.986 5.128824) (end -13.5025 6.612324) (width 0.25) (layer "F.Cu") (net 1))
 (segment (start -15 1.025) (end -13.471 1.025) (width 0.25) (layer "F.Cu") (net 1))
 (segment (start -15 3.796) (end -14.986 3.81) (width 0.25) (layer "F.Cu") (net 1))
 (segment (start -15 1.025) (end -15 3.796) (width 0.25) (layer "F.Cu") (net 1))
 (segment (start -13.5025 6.612324) (end -14.224 7.333824) (width 0.25) (layer "F.Cu") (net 1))
 (segment (start 15 1.025) (end 13.979 1.025) (width 0.25) (layer "F.Cu") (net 1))
 (segment (start -12.4775 -8.387676) (end -10.934912 -6.845088) (width 0.25) (layer "F.Cu") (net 1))
 (via (at 13.97 1.016) (size 0.8) (drill 0.4) (layers "F.Cu" "B.Cu") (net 1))
 (via (at -13.462 1.016) (size 0.8) (drill 0.4) (layers "F.Cu" "B.Cu") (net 1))
 (via (at -7.112 -12.192) (size 0.8) (drill 0.4) (layers "F.Cu" "B.Cu") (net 1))
 (via (at -10.934912 -6.845088) (size 0.8) (drill 0.4) (layers "F.Cu" "B.Cu") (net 1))
 (segment (start 5.328728 -12.192) (end -7.112 -12.192) (width 0.25) (layer "B.Cu") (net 1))
 (segment (start 13.97 -3.550728) (end 5.328728 -12.192) (width 0.25) (layer "B.Cu") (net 1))
 (segment (start 13.97 1.016) (end 13.97 -3.550728) (width 0.25) (layer "B.Cu") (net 1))
 (segment (start -10.934912 -1.511088) (end -13.462 1.016) (width 0.25) (layer "B.Cu") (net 1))
 (segment (start -10.934912 -6.845088) (end -10.934912 -1.511088) (width 0.25) (layer "B.Cu") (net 1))
 (segment (start -6.387 -11.901) (end -6.387 -11.891695) (width 0.25) (layer "F.Cu") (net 7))
 (segment (start -8.387676 12.4775) (end -7.848176 11.938) (width 0.25) (layer "F.Cu") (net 7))
 (segment (start 1.025 -15) (end -0.513 -13.462) (width 0.25) (layer "F.Cu") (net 7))
 (segment (start 8.247486 14.224) (end 13.97 8.501486) (width 0.25) (layer "F.Cu") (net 7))
 (segment (start 13.97 8.501486) (end 13.97 7.079824) (width 0.25) (layer "F.Cu") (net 7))
 (segment (start -12.4775 8.387676) (end -12.451676 8.387676) (width 0.25) (layer "F.Cu") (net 7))
 (segment (start -7.848176 11.938) (end -6.096 11.938) (width 0.25) (layer "F.Cu") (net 7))
 (segment (start -0.513 -13.462) (end -4.826 -13.462) (width 0.25) (layer "F.Cu") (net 7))
 (segment (start -12.451676 8.387676) (end -11.684 7.62) (width 0.25) (layer "F.Cu") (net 7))
 (segment (start -6.821 -11.467) (end -9.652 -8.636) (width 0.25) (layer "F.Cu") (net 7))
 (segment (start -0.259 13.716) (end 1.025 15) (width 0.25) (layer "F.Cu") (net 7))
 (segment (start -9.652 -8.636) (end -9.652 -7.366) (width 0.25) (layer "F.Cu") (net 7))
 (segment (start -4.826 -13.462) (end -6.387 -11.901) (width 0.25) (layer "F.Cu") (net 7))
 (segment (start 7.333824 14.224) (end 8.247486 14.224) (width 0.25) (layer "F.Cu") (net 7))
 (segment (start 1.025 15) (end 5.114824 15) (width 0.25) (layer "F.Cu") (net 7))
 (segment (start -6.811695 -11.467) (end -6.821 -11.467) (width 0.25) (layer "F.Cu") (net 7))
 (segment (start 6.612324 13.5025) (end 7.333824 14.224) (width 0.25) (layer "F.Cu") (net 7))
 (segment (start -8.636 -6.35) (end -6.842 -6.35) (width 0.25) (layer "F.Cu") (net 7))
 (segment (start -4.318 13.716) (end -0.259 13.716) (width 0.25) (layer "F.Cu") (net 7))
 (segment (start 5.114824 15) (end 6.612324 13.5025) (width 0.25) (layer "F.Cu") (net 7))
 (segment (start -6.387 -11.891695) (end -6.811695 -11.467) (width 0.25) (layer "F.Cu") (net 7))
 (segment (start -6.096 11.938) (end -4.318 13.716) (width 0.25) (layer "F.Cu") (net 7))
 (segment (start -9.652 -7.366) (end -8.636 -6.35) (width 0.25) (layer "F.Cu") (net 7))
 (segment (start 13.97 7.079824) (end 13.5025 6.612324) (width 0.25) (layer "F.Cu") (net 7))
 (segment (start -12.4775 8.387676) (end -8.387676 12.4775) (width 0.25) (layer "F.Cu") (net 7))
 (via (at -9.652 -7.366) (size 0.8) (drill 0.4) (layers "F.Cu" "B.Cu") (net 7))
 (via (at -11.684 7.62) (size 0.8) (drill 0.4) (layers "F.Cu" "B.Cu") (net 7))
 (segment (start -9.906 -7.112) (end -9.652 -7.366) (width 0.25) (layer "B.Cu") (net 7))
 (segment (start -11.684 7.62) (end -11.684 0.254) (width 0.25) (layer "B.Cu") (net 7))
 (segment (start -11.684 0.254) (end -9.906 -1.524) (width 0.25) (layer "B.Cu") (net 7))
 (segment (start -9.906 -1.524) (end -9.906 -7.112) (width 0.25) (layer "B.Cu") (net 7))
 (segment (start 0 0) (end 2.475 0) (width 0.25) (layer "F.Cu") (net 17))
 (segment (start -4.842 -6.35) (end -3.556 -6.35) (width 0.25) (layer "F.Cu") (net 17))
 (via (at 0 0) (size 0.8) (drill 0.4) (layers "F.Cu" "B.Cu") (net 17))
 (via (at -3.556 -6.35) (size 0.8) (drill 0.4) (layers "F.Cu" "B.Cu") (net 17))
 (segment (start 0 0) (end -3.556 -3.556) (width 0.25) (layer "B.Cu") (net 17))
 (segment (start -3.556 -3.556) (end -3.556 -6.35) (width 0.25) (layer "B.Cu") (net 17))
 (segment (start -3.064 -2.54) (end -4.842 -4.318) (width 0.25) (layer "F.Cu") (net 6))
 (segment (start -2.475 -2.54) (end -3.064 -2.54) (width 0.25) (layer "F.Cu") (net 6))
 (segment (start -2.475 -1.27) (end -3.826 -1.27) (width 0.25) (layer "F.Cu") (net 9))
 (segment (start -3.826 -1.27) (end -4.842 -2.286) (width 0.25) (layer "F.Cu") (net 9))
 (segment (start -2.475 0) (end -4.588 0) (width 0.25) (layer "F.Cu") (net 10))
 (segment (start -4.588 0) (end -4.842 -0.254) (width 0.25) (layer "F.Cu") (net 10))
 (segment (start 3.81 -7.366) (end 3.81 1.27) (width 0.25) (layer "F.Cu") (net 16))
 (segment (start 3.81 1.27) (end 2.475 1.27) (width 0.25) (layer "F.Cu") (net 16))
 (segment (start 1.025001 5.324999) (end 1.421999 5.324999) (width 0.25) (layer "F.Cu") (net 3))
 (segment (start 1.421999 5.324999) (end 2.625 6.528) (width 0.25) (layer "F.Cu") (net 3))
 (segment (start -2.625 6.528) (end 2.625 6.528) (width 0.25) (layer "F.Cu") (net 3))
 (segment (start 2.475 -1.27) (end 1.016 -1.27) (width 0.25) (layer "F.Cu") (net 3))
 (via (at 1.016 -1.27) (size 0.8) (drill 0.4) (layers "F.Cu" "B.Cu") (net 3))
 (via (at 1.025001 5.324999) (size 0.8) (drill 0.4) (layers "F.Cu" "B.Cu") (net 3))
 (segment (start 1.025001 -1.260999) (end 1.025001 5.324999) (width 0.25) (layer "B.Cu") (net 3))
 (segment (start 1.016 -1.27) (end 1.025001 -1.260999) (width 0.25) (layer "B.Cu") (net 3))
 (segment (start 10.204 2.5) (end 5.7 2.5) (width 0.25) (layer "B.Cu") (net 19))
 (segment (start 5.7 2.5) (end 0 8.2) (width 0.25) (layer "B.Cu") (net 19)))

